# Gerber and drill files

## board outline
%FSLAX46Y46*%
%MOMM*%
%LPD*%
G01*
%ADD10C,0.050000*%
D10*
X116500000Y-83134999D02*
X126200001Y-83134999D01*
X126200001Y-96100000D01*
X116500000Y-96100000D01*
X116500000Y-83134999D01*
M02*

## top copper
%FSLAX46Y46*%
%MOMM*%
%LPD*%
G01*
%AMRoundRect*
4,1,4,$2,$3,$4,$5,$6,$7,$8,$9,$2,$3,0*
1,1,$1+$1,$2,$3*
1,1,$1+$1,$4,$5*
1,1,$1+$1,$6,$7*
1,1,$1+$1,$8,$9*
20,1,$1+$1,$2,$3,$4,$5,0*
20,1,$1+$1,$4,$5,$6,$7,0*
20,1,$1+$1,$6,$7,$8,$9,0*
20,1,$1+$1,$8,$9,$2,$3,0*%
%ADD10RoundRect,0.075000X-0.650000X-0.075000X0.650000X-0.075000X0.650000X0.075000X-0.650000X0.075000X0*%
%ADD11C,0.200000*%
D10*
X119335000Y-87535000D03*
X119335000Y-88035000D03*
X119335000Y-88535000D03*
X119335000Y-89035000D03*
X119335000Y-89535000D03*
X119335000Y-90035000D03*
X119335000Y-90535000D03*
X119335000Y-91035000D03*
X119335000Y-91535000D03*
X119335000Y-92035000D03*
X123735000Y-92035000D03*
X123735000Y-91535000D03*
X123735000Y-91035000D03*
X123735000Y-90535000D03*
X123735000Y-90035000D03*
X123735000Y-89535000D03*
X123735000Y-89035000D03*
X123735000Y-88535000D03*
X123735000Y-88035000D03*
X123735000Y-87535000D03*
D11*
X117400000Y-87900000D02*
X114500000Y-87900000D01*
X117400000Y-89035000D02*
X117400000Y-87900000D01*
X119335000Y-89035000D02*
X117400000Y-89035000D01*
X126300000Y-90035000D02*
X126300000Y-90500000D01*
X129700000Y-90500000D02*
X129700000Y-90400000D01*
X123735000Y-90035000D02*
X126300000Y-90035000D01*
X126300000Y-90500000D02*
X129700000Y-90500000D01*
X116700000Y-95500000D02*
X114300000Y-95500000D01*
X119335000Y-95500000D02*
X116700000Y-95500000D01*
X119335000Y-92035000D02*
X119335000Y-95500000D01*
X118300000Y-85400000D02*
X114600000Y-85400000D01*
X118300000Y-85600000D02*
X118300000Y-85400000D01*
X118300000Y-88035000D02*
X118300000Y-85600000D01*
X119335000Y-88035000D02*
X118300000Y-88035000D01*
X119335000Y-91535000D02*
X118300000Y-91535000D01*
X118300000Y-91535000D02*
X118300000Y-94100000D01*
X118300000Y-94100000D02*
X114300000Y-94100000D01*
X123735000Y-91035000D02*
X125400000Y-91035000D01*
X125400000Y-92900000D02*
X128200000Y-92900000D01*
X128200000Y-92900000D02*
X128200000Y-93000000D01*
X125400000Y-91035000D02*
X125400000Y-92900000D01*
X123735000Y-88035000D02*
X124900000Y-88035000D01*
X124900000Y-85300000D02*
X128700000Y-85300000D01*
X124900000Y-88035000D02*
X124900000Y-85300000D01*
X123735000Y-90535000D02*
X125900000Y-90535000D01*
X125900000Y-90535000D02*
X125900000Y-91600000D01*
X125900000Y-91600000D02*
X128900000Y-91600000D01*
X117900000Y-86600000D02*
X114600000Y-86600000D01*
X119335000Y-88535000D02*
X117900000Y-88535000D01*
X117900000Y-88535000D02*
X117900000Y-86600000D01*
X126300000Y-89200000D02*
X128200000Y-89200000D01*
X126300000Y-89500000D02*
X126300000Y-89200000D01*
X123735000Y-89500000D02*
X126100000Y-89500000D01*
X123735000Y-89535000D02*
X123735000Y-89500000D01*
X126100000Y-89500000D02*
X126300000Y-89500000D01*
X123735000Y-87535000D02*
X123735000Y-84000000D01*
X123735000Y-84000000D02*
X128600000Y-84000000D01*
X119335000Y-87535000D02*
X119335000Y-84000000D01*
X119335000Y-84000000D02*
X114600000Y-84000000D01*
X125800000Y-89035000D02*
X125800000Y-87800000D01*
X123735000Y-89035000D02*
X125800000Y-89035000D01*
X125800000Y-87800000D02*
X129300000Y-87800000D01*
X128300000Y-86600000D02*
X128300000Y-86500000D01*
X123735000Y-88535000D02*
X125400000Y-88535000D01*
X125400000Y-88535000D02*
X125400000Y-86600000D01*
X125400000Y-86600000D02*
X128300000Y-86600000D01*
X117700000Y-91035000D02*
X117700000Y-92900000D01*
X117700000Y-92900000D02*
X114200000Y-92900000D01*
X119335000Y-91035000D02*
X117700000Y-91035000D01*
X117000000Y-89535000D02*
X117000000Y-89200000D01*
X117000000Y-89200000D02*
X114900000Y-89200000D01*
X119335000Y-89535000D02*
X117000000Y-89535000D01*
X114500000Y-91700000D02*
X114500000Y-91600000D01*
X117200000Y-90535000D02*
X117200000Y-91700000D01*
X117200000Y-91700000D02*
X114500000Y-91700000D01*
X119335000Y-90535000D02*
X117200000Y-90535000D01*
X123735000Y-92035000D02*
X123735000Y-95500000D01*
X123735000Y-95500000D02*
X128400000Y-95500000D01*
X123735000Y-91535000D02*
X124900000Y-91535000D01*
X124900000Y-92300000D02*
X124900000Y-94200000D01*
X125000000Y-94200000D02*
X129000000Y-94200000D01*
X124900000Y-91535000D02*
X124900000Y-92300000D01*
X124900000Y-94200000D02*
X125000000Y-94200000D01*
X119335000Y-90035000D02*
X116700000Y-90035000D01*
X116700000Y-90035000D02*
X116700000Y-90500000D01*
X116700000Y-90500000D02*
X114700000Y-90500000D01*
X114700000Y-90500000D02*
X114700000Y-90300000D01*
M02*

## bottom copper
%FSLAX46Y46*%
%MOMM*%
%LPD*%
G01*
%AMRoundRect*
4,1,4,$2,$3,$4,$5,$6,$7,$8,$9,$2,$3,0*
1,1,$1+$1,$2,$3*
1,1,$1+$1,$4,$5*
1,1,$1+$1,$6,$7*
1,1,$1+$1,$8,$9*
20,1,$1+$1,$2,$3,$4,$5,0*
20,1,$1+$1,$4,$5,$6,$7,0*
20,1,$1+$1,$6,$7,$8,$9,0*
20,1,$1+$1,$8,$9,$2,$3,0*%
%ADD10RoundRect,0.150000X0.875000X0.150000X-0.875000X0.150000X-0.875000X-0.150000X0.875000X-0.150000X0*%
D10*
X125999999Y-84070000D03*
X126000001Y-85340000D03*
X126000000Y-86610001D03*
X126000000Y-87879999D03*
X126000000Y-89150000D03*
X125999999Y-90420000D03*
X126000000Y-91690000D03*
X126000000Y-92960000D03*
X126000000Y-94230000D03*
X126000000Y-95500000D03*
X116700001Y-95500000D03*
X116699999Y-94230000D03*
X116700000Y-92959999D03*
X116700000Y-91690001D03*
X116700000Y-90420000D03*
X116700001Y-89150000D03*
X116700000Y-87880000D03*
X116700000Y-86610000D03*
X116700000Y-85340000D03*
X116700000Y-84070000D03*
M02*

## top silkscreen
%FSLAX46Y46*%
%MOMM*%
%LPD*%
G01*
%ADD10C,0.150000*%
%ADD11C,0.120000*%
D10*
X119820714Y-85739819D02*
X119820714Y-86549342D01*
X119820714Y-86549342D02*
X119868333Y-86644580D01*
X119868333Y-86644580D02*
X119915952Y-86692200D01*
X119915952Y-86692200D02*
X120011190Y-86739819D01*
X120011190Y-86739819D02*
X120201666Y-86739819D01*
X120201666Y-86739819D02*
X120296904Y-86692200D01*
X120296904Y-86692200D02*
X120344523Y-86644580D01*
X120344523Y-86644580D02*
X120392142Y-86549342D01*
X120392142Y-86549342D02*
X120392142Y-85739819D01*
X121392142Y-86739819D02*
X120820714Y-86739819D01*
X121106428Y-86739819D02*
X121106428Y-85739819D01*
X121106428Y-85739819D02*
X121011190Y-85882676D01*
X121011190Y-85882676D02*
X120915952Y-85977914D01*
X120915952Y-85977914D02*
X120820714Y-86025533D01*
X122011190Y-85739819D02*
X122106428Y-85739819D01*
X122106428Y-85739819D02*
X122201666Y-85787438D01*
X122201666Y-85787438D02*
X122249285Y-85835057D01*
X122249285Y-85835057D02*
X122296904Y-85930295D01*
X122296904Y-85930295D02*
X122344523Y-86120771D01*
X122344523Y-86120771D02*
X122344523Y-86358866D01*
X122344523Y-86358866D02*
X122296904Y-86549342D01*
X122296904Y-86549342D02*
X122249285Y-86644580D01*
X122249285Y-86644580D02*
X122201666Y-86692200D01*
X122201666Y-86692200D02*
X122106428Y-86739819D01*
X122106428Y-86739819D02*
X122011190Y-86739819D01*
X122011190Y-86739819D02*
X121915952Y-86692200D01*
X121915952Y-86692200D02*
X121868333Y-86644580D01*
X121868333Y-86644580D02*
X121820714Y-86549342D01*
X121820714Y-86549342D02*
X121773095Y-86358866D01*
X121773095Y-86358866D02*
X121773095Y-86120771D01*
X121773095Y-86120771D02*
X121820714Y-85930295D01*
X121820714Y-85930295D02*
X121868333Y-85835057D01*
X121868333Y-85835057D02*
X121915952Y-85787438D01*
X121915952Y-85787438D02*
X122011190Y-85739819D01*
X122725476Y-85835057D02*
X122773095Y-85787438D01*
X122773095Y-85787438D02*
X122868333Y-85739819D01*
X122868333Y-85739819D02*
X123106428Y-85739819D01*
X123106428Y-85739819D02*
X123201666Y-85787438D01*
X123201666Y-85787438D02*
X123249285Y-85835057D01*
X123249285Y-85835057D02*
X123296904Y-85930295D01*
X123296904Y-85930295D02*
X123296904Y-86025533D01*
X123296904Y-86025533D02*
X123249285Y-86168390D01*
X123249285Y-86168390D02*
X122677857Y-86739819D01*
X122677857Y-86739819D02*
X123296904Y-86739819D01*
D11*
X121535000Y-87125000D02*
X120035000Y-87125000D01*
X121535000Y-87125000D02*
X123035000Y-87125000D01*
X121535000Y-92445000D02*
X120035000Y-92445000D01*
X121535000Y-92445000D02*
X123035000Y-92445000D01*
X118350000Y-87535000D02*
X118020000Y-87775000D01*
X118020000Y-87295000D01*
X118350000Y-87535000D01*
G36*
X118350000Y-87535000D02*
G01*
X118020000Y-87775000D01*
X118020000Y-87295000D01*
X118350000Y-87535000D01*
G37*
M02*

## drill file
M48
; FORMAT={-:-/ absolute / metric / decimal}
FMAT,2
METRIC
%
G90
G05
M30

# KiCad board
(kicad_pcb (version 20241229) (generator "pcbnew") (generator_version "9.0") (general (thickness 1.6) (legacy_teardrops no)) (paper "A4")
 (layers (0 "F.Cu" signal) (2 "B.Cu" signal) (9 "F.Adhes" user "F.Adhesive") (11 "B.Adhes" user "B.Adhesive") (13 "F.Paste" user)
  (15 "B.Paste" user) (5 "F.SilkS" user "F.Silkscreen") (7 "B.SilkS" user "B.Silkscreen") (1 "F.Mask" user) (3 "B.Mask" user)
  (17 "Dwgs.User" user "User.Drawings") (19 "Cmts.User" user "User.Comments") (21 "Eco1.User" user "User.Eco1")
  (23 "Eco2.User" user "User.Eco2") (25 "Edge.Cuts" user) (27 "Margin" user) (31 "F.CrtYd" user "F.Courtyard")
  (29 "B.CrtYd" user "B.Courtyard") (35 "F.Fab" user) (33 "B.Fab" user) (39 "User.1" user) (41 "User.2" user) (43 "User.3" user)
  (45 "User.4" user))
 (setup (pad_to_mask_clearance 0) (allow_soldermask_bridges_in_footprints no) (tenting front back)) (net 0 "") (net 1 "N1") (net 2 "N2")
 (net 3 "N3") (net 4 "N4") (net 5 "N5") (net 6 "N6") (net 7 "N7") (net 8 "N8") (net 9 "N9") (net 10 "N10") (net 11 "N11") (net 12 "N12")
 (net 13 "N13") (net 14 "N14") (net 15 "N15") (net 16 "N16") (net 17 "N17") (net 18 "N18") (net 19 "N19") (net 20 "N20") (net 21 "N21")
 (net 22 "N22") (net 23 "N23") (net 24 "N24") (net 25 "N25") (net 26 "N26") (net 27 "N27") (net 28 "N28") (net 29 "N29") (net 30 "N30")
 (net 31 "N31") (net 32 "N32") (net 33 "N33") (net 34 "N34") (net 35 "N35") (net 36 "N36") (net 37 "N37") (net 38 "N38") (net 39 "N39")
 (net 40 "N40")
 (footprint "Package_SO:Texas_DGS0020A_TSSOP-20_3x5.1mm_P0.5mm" (layer "F.Cu") (at 121.535 89.785)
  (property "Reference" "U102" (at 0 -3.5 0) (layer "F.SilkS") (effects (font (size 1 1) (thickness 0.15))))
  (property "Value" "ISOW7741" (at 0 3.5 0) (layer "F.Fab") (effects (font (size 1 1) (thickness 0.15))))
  (fp_line (start 0 -2.66) (end -1.5 -2.66) (stroke (width 0.12) (type solid)) (layer "F.SilkS"))
  (fp_line (start 0 -2.66) (end 1.5 -2.66) (stroke (width 0.12) (type solid)) (layer "F.SilkS"))
  (fp_line (start 0 2.66) (end -1.5 2.66) (stroke (width 0.12) (type solid)) (layer "F.SilkS"))
  (fp_line (start 0 2.66) (end 1.5 2.66) (stroke (width 0.12) (type solid)) (layer "F.SilkS"))
  (fp_poly (pts (xy -3.185 -2.25) (xy -3.515 -2.01) (xy -3.515 -2.49)) (stroke (width 0.12) (type solid)) (fill yes) (layer "F.SilkS"))
  (pad "1" smd roundrect (at -2.2 -2.25) (size 1.45 0.3) (layers "F.Cu" "F.Mask" "F.Paste") (roundrect_rratio 0.25) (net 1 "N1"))
  (pad "2" smd roundrect (at -2.2 -1.75) (size 1.45 0.3) (layers "F.Cu" "F.Mask" "F.Paste") (roundrect_rratio 0.25) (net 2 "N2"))
  (pad "3" smd roundrect (at -2.2 -1.25) (size 1.45 0.3) (layers "F.Cu" "F.Mask" "F.Paste") (roundrect_rratio 0.25) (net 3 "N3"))
  (pad "4" smd roundrect (at -2.2 -0.75) (size 1.45 0.3) (layers "F.Cu" "F.Mask" "F.Paste") (roundrect_rratio 0.25) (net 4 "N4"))
  (pad "5" smd roundrect (at -2.2 -0.25) (size 1.45 0.3) (layers "F.Cu" "F.Mask" "F.Paste") (roundrect_rratio 0.25) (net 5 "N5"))
  (pad "6" smd roundrect (at -2.2 0.25) (size 1.45 0.3) (layers "F.Cu" "F.Mask" "F.Paste") (roundrect_rratio 0.25) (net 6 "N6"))
  (pad "7" smd roundrect (at -2.2 0.75) (size 1.45 0.3) (layers "F.Cu" "F.Mask" "F.Paste") (roundrect_rratio 0.25) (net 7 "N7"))
  (pad "8" smd roundrect (at -2.2 1.25) (size 1.45 0.3) (layers "F.Cu" "F.Mask" "F.Paste") (roundrect_rratio 0.25) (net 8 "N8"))
  (pad "9" smd roundrect (at -2.2 1.75) (size 1.45 0.3) (layers "F.Cu" "F.Mask" "F.Paste") (roundrect_rratio 0.25) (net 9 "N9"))
  (pad "10" smd roundrect (at -2.2 2.25) (size 1.45 0.3) (layers "F.Cu" "F.Mask" "F.Paste") (roundrect_rratio 0.25) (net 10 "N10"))
  (pad "11" smd roundrect (at 2.2 2.25) (size 1.45 0.3) (layers "F.Cu" "F.Mask" "F.Paste") (roundrect_rratio 0.25) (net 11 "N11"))
  (pad "12" smd roundrect (at 2.2 1.75) (size 1.45 0.3) (layers "F.Cu" "F.Mask" "F.Paste") (roundrect_rratio 0.25) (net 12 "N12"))
  (pad "13" smd roundrect (at 2.2 1.25) (size 1.45 0.3) (layers "F.Cu" "F.Mask" "F.Paste") (roundrect_rratio 0.25) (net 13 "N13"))
  (pad "14" smd roundrect (at 2.2 0.75) (size 1.45 0.3) (layers "F.Cu" "F.Mask" "F.Paste") (roundrect_rratio 0.25) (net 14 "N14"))
  (pad "15" smd roundrect (at 2.2 0.25) (size 1.45 0.3) (layers "F.Cu" "F.Mask" "F.Paste") (roundrect_rratio 0.25) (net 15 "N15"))
  (pad "16" smd roundrect (at 2.2 -0.25) (size 1.45 0.3) (layers "F.Cu" "F.Mask" "F.Paste") (roundrect_rratio 0.25) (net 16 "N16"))
  (pad "17" smd roundrect (at 2.2 -0.75) (size 1.45 0.3) (layers "F.Cu" "F.Mask" "F.Paste") (roundrect_rratio 0.25) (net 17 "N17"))
  (pad "18" smd roundrect (at 2.2 -1.25) (size 1.45 0.3) (layers "F.Cu" "F.Mask" "F.Paste") (roundrect_rratio 0.25) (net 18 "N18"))
  (pad "19" smd roundrect (at 2.2 -1.75) (size 1.45 0.3) (layers "F.Cu" "F.Mask" "F.Paste") (roundrect_rratio 0.25) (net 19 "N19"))
  (pad "20" smd roundrect (at 2.2 -2.25) (size 1.45 0.3) (layers "F.Cu" "F.Mask" "F.Paste") (roundrect_rratio 0.25) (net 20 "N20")))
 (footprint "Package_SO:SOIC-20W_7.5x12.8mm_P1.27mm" (layer "B.Cu") (at 121.35 89.785 180)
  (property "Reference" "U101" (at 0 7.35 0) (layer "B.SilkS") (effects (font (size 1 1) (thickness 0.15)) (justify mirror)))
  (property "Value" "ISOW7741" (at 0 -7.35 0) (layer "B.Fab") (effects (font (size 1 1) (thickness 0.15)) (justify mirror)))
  (pad "1" smd roundrect (at -4.649999 5.715 180) (size 2.05 0.6) (layers "B.Cu" "B.Mask" "B.Paste") (roundrect_rratio 0.25) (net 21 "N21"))
  (pad "2" smd roundrect (at -4.650001 4.445 180) (size 2.05 0.6) (layers "B.Cu" "B.Mask" "B.Paste") (roundrect_rratio 0.25) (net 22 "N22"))
  (pad "3" smd roundrect (at -4.65 3.174999 180) (size 2.05 0.6) (layers "B.Cu" "B.Mask" "B.Paste") (roundrect_rratio 0.25) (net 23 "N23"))
  (pad "4" smd roundrect (at -4.65 1.905001 180) (size 2.05 0.6) (layers "B.Cu" "B.Mask" "B.Paste") (roundrect_rratio 0.25) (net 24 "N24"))
  (pad "5" smd roundrect (at -4.65 0.635 180) (size 2.05 0.6) (layers "B.Cu" "B.Mask" "B.Paste") (roundrect_rratio 0.25) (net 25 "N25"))
  (pad "6" smd roundrect (at -4.649999 -0.635 180) (size 2.05 0.6) (layers "B.Cu" "B.Mask" "B.Paste") (roundrect_rratio 0.25) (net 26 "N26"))
  (pad "7" smd roundrect (at -4.65 -1.905 180) (size 2.05 0.6) (layers "B.Cu" "B.Mask" "B.Paste") (roundrect_rratio 0.25) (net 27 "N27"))
  (pad "8" smd roundrect (at -4.65 -3.175 180) (size 2.05 0.6) (layers "B.Cu" "B.Mask" "B.Paste") (roundrect_rratio 0.25) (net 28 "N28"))
  (pad "9" smd roundrect (at -4.65 -4.445 180) (size 2.05 0.6) (layers "B.Cu" "B.Mask" "B.Paste") (roundrect_rratio 0.25) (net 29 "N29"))
  (pad "10" smd roundrect (at -4.65 -5.715 180) (size 2.05 0.6) (layers "B.Cu" "B.Mask" "B.Paste") (roundrect_rratio 0.25) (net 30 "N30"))
  (pad "11" smd roundrect (at 4.649999 -5.715 180) (size 2.05 0.6) (layers "B.Cu" "B.Mask" "B.Paste") (roundrect_rratio 0.25) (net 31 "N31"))
  (pad "12" smd roundrect (at 4.650001 -4.445 180) (size 2.05 0.6) (layers "B.Cu" "B.Mask" "B.Paste") (roundrect_rratio 0.25) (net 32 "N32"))
  (pad "13" smd roundrect (at 4.65 -3.174999 180) (size 2.05 0.6) (layers "B.Cu" "B.Mask" "B.Paste") (roundrect_rratio 0.25) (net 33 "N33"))
  (pad "14" smd roundrect (at 4.65 -1.905001 180) (size 2.05 0.6) (layers "B.Cu" "B.Mask" "B.Paste") (roundrect_rratio 0.25) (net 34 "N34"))
  (pad "15" smd roundrect (at 4.65 -0.635 180) (size 2.05 0.6) (layers "B.Cu" "B.Mask" "B.Paste") (roundrect_rratio 0.25) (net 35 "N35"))
  (pad "16" smd roundrect (at 4.649999 0.635 180) (size 2.05 0.6) (layers "B.Cu" "B.Mask" "B.Paste") (roundrect_rratio 0.25) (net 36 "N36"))
  (pad "17" smd roundrect (at 4.65 1.905 180) (size 2.05 0.6) (layers "B.Cu" "B.Mask" "B.Paste") (roundrect_rratio 0.25) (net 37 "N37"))
  (pad "18" smd roundrect (at 4.65 3.175 180) (size 2.05 0.6) (layers "B.Cu" "B.Mask" "B.Paste") (roundrect_rratio 0.25) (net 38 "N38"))
  (pad "19" smd roundrect (at 4.65 4.445 180) (size 2.05 0.6) (layers "B.Cu" "B.Mask" "B.Paste") (roundrect_rratio 0.25) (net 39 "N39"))
  (pad "20" smd roundrect (at 4.65 5.715 180) (size 2.05 0.6) (layers "B.Cu" "B.Mask" "B.Paste") (roundrect_rratio 0.25) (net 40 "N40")))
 (gr_rect (start 116.5 83.134999) (end 126.200001 96.1) (stroke (width 0.05) (type default)) (fill no) (layer "Edge.Cuts"))
 (segment (start 117.4 87.9) (end 114.5 87.9) (width 0.2) (layer "F.Cu") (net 4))
 (segment (start 117.4 89.035) (end 117.4 87.9) (width 0.2) (layer "F.Cu") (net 4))
 (segment (start 119.335 89.035) (end 117.4 89.035) (width 0.2) (layer "F.Cu") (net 4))
 (segment (start 126.3 90.035) (end 126.3 90.5) (width 0.2) (layer "F.Cu") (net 15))
 (segment (start 129.7 90.5) (end 129.7 90.4) (width 0.2) (layer "F.Cu") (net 15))
 (segment (start 123.735 90.035) (end 126.3 90.035) (width 0.2) (layer "F.Cu") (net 15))
 (segment (start 126.3 90.5) (end 129.7 90.5) (width 0.2) (layer "F.Cu") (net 15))
 (segment (start 116.7 95.5) (end 114.3 95.5) (width 0.2) (layer "F.Cu") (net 10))
 (segment (start 119.335 95.5) (end 116.7 95.5) (width 0.2) (layer "F.Cu") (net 10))
 (segment (start 119.335 92.035) (end 119.335 95.5) (width 0.2) (layer "F.Cu") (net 10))
 (segment (start 118.3 85.4) (end 114.6 85.4) (width 0.2) (layer "F.Cu") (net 2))
 (segment (start 118.3 85.6) (end 118.3 85.4) (width 0.2) (layer "F.Cu") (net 2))
 (segment (start 118.3 88.035) (end 118.3 85.6) (width 0.2) (layer "F.Cu") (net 2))
 (segment (start 119.335 88.035) (end 118.3 88.035) (width 0.2) (layer "F.Cu") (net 2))
 (segment (start 119.335 91.535) (end 118.3 91.535) (width 0.2) (layer "F.Cu") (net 9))
 (segment (start 118.3 91.535) (end 118.3 94.1) (width 0.2) (layer "F.Cu") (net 9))
 (segment (start 118.3 94.1) (end 114.3 94.1) (width 0.2) (layer "F.Cu") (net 9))
 (segment (start 123.735 91.035) (end 125.4 91.035) (width 0.2) (layer "F.Cu") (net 13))
 (segment (start 125.4 92.9) (end 128.2 92.9) (width 0.2) (layer "F.Cu") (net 13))
 (segment (start 128.2 92.9) (end 128.2 93) (width 0.2) (layer "F.Cu") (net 13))
 (segment (start 125.4 91.035) (end 125.4 92.9) (width 0.2) (layer "F.Cu") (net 13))
 (segment (start 123.735 88.035) (end 124.9 88.035) (width 0.2) (layer "F.Cu") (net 19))
 (segment (start 124.9 85.3) (end 128.7 85.3) (width 0.2) (layer "F.Cu") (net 19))
 (segment (start 124.9 88.035) (end 124.9 85.3) (width 0.2) (layer "F.Cu") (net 19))
 (segment (start 123.735 90.535) (end 125.9 90.535) (width 0.2) (layer "F.Cu") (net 14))
 (segment (start 125.9 90.535) (end 125.9 91.6) (width 0.2) (layer "F.Cu") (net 14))
 (segment (start 125.9 91.6) (end 128.9 91.6) (width 0.2) (layer "F.Cu") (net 14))
 (segment (start 117.9 86.6) (end 114.6 86.6) (width 0.2) (layer "F.Cu") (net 3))
 (segment (start 119.335 88.535) (end 117.9 88.535) (width 0.2) (layer "F.Cu") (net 3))
 (segment (start 117.9 88.535) (end 117.9 86.6) (width 0.2) (layer "F.Cu") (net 3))
 (segment (start 126.3 89.2) (end 128.2 89.2) (width 0.2) (layer "F.Cu") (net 16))
 (segment (start 126.3 89.5) (end 126.3 89.2) (width 0.2) (layer "F.Cu") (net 16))
 (segment (start 123.735 89.5) (end 126.1 89.5) (width 0.2) (layer "F.Cu") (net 16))
 (segment (start 123.735 89.535) (end 123.735 89.5) (width 0.2) (layer "F.Cu") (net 16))
 (segment (start 126.1 89.5) (end 126.3 89.5) (width 0.2) (layer "F.Cu") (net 16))
 (segment (start 123.735 87.535) (end 123.735 84) (width 0.2) (layer "F.Cu") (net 20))
 (segment (start 123.735 84) (end 128.6 84) (width 0.2) (layer "F.Cu") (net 20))
 (segment (start 119.335 87.535) (end 119.335 84) (width 0.2) (layer "F.Cu") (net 1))
 (segment (start 119.335 84) (end 114.6 84) (width 0.2) (layer "F.Cu") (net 1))
 (segment (start 125.8 89.035) (end 125.8 87.8) (width 0.2) (layer "F.Cu") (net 17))
 (segment (start 123.735 89.035) (end 125.8 89.035) (width 0.2) (layer "F.Cu") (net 17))
 (segment (start 125.8 87.8) (end 129.3 87.8) (width 0.2) (layer "F.Cu") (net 17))
 (segment (start 128.3 86.6) (end 128.3 86.5) (width 0.2) (layer "F.Cu") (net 18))
 (segment (start 123.735 88.535) (end 125.4 88.535) (width 0.2) (layer "F.Cu") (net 18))
 (segment (start 125.4 88.535) (end 125.4 86.6) (width 0.2) (layer "F.Cu") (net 18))
 (segment (start 125.4 86.6) (end 128.3 86.6) (width 0.2) (layer "F.Cu") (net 18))
 (segment (start 117.7 91.035) (end 117.7 92.9) (width 0.2) (layer "F.Cu") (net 8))
 (segment (start 117.7 92.9) (end 114.2 92.9) (width 0.2) (layer "F.Cu") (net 8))
 (segment (start 119.335 91.035) (end 117.7 91.035) (width 0.2) (layer "F.Cu") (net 8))
 (segment (start 117 89.535) (end 117 89.2) (width 0.2) (layer "F.Cu") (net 5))
 (segment (start 117 89.2) (end 114.9 89.2) (width 0.2) (layer "F.Cu") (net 5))
 (segment (start 119.335 89.535) (end 117 89.535) (width 0.2) (layer "F.Cu") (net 5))
 (segment (start 114.5 91.7) (end 114.5 91.6) (width 0.2) (layer "F.Cu") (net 7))
 (segment (start 117.2 90.535) (end 117.2 91.7) (width 0.2) (layer "F.Cu") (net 7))
 (segment (start 117.2 91.7) (end 114.5 91.7) (width 0.2) (layer "F.Cu") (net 7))
 (segment (start 119.335 90.535) (end 117.2 90.535) (width 0.2) (layer "F.Cu") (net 7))
 (segment (start 123.735 92.035) (end 123.735 95.5) (width 0.2) (layer "F.Cu") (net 11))
 (segment (start 123.735 95.5) (end 128.4 95.5) (width 0.2) (layer "F.Cu") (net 11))
 (segment (start 123.735 91.535) (end 124.9 91.535) (width 0.2) (layer "F.Cu") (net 12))
 (segment (start 124.9 92.3) (end 124.9 94.2) (width 0.2) (layer "F.Cu") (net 12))
 (segment (start 125 94.2) (end 129 94.2) (width 0.2) (layer "F.Cu") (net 12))
 (segment (start 124.9 91.535) (end 124.9 92.3) (width 0.2) (layer "F.Cu") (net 12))
 (segment (start 124.9 94.2) (end 125 94.2) (width 0.2) (layer "F.Cu") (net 12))
 (segment (start 119.335 90.035) (end 116.7 90.035) (width 0.2) (layer "F.Cu") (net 6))
 (segment (start 116.7 90.035) (end 116.7 90.5) (width 0.2) (layer "F.Cu") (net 6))
 (segment (start 116.7 90.5) (end 114.7 90.5) (width 0.2) (layer "F.Cu") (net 6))
 (segment (start 114.7 90.5) (end 114.7 90.3) (width 0.2) (layer "F.Cu") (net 6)))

